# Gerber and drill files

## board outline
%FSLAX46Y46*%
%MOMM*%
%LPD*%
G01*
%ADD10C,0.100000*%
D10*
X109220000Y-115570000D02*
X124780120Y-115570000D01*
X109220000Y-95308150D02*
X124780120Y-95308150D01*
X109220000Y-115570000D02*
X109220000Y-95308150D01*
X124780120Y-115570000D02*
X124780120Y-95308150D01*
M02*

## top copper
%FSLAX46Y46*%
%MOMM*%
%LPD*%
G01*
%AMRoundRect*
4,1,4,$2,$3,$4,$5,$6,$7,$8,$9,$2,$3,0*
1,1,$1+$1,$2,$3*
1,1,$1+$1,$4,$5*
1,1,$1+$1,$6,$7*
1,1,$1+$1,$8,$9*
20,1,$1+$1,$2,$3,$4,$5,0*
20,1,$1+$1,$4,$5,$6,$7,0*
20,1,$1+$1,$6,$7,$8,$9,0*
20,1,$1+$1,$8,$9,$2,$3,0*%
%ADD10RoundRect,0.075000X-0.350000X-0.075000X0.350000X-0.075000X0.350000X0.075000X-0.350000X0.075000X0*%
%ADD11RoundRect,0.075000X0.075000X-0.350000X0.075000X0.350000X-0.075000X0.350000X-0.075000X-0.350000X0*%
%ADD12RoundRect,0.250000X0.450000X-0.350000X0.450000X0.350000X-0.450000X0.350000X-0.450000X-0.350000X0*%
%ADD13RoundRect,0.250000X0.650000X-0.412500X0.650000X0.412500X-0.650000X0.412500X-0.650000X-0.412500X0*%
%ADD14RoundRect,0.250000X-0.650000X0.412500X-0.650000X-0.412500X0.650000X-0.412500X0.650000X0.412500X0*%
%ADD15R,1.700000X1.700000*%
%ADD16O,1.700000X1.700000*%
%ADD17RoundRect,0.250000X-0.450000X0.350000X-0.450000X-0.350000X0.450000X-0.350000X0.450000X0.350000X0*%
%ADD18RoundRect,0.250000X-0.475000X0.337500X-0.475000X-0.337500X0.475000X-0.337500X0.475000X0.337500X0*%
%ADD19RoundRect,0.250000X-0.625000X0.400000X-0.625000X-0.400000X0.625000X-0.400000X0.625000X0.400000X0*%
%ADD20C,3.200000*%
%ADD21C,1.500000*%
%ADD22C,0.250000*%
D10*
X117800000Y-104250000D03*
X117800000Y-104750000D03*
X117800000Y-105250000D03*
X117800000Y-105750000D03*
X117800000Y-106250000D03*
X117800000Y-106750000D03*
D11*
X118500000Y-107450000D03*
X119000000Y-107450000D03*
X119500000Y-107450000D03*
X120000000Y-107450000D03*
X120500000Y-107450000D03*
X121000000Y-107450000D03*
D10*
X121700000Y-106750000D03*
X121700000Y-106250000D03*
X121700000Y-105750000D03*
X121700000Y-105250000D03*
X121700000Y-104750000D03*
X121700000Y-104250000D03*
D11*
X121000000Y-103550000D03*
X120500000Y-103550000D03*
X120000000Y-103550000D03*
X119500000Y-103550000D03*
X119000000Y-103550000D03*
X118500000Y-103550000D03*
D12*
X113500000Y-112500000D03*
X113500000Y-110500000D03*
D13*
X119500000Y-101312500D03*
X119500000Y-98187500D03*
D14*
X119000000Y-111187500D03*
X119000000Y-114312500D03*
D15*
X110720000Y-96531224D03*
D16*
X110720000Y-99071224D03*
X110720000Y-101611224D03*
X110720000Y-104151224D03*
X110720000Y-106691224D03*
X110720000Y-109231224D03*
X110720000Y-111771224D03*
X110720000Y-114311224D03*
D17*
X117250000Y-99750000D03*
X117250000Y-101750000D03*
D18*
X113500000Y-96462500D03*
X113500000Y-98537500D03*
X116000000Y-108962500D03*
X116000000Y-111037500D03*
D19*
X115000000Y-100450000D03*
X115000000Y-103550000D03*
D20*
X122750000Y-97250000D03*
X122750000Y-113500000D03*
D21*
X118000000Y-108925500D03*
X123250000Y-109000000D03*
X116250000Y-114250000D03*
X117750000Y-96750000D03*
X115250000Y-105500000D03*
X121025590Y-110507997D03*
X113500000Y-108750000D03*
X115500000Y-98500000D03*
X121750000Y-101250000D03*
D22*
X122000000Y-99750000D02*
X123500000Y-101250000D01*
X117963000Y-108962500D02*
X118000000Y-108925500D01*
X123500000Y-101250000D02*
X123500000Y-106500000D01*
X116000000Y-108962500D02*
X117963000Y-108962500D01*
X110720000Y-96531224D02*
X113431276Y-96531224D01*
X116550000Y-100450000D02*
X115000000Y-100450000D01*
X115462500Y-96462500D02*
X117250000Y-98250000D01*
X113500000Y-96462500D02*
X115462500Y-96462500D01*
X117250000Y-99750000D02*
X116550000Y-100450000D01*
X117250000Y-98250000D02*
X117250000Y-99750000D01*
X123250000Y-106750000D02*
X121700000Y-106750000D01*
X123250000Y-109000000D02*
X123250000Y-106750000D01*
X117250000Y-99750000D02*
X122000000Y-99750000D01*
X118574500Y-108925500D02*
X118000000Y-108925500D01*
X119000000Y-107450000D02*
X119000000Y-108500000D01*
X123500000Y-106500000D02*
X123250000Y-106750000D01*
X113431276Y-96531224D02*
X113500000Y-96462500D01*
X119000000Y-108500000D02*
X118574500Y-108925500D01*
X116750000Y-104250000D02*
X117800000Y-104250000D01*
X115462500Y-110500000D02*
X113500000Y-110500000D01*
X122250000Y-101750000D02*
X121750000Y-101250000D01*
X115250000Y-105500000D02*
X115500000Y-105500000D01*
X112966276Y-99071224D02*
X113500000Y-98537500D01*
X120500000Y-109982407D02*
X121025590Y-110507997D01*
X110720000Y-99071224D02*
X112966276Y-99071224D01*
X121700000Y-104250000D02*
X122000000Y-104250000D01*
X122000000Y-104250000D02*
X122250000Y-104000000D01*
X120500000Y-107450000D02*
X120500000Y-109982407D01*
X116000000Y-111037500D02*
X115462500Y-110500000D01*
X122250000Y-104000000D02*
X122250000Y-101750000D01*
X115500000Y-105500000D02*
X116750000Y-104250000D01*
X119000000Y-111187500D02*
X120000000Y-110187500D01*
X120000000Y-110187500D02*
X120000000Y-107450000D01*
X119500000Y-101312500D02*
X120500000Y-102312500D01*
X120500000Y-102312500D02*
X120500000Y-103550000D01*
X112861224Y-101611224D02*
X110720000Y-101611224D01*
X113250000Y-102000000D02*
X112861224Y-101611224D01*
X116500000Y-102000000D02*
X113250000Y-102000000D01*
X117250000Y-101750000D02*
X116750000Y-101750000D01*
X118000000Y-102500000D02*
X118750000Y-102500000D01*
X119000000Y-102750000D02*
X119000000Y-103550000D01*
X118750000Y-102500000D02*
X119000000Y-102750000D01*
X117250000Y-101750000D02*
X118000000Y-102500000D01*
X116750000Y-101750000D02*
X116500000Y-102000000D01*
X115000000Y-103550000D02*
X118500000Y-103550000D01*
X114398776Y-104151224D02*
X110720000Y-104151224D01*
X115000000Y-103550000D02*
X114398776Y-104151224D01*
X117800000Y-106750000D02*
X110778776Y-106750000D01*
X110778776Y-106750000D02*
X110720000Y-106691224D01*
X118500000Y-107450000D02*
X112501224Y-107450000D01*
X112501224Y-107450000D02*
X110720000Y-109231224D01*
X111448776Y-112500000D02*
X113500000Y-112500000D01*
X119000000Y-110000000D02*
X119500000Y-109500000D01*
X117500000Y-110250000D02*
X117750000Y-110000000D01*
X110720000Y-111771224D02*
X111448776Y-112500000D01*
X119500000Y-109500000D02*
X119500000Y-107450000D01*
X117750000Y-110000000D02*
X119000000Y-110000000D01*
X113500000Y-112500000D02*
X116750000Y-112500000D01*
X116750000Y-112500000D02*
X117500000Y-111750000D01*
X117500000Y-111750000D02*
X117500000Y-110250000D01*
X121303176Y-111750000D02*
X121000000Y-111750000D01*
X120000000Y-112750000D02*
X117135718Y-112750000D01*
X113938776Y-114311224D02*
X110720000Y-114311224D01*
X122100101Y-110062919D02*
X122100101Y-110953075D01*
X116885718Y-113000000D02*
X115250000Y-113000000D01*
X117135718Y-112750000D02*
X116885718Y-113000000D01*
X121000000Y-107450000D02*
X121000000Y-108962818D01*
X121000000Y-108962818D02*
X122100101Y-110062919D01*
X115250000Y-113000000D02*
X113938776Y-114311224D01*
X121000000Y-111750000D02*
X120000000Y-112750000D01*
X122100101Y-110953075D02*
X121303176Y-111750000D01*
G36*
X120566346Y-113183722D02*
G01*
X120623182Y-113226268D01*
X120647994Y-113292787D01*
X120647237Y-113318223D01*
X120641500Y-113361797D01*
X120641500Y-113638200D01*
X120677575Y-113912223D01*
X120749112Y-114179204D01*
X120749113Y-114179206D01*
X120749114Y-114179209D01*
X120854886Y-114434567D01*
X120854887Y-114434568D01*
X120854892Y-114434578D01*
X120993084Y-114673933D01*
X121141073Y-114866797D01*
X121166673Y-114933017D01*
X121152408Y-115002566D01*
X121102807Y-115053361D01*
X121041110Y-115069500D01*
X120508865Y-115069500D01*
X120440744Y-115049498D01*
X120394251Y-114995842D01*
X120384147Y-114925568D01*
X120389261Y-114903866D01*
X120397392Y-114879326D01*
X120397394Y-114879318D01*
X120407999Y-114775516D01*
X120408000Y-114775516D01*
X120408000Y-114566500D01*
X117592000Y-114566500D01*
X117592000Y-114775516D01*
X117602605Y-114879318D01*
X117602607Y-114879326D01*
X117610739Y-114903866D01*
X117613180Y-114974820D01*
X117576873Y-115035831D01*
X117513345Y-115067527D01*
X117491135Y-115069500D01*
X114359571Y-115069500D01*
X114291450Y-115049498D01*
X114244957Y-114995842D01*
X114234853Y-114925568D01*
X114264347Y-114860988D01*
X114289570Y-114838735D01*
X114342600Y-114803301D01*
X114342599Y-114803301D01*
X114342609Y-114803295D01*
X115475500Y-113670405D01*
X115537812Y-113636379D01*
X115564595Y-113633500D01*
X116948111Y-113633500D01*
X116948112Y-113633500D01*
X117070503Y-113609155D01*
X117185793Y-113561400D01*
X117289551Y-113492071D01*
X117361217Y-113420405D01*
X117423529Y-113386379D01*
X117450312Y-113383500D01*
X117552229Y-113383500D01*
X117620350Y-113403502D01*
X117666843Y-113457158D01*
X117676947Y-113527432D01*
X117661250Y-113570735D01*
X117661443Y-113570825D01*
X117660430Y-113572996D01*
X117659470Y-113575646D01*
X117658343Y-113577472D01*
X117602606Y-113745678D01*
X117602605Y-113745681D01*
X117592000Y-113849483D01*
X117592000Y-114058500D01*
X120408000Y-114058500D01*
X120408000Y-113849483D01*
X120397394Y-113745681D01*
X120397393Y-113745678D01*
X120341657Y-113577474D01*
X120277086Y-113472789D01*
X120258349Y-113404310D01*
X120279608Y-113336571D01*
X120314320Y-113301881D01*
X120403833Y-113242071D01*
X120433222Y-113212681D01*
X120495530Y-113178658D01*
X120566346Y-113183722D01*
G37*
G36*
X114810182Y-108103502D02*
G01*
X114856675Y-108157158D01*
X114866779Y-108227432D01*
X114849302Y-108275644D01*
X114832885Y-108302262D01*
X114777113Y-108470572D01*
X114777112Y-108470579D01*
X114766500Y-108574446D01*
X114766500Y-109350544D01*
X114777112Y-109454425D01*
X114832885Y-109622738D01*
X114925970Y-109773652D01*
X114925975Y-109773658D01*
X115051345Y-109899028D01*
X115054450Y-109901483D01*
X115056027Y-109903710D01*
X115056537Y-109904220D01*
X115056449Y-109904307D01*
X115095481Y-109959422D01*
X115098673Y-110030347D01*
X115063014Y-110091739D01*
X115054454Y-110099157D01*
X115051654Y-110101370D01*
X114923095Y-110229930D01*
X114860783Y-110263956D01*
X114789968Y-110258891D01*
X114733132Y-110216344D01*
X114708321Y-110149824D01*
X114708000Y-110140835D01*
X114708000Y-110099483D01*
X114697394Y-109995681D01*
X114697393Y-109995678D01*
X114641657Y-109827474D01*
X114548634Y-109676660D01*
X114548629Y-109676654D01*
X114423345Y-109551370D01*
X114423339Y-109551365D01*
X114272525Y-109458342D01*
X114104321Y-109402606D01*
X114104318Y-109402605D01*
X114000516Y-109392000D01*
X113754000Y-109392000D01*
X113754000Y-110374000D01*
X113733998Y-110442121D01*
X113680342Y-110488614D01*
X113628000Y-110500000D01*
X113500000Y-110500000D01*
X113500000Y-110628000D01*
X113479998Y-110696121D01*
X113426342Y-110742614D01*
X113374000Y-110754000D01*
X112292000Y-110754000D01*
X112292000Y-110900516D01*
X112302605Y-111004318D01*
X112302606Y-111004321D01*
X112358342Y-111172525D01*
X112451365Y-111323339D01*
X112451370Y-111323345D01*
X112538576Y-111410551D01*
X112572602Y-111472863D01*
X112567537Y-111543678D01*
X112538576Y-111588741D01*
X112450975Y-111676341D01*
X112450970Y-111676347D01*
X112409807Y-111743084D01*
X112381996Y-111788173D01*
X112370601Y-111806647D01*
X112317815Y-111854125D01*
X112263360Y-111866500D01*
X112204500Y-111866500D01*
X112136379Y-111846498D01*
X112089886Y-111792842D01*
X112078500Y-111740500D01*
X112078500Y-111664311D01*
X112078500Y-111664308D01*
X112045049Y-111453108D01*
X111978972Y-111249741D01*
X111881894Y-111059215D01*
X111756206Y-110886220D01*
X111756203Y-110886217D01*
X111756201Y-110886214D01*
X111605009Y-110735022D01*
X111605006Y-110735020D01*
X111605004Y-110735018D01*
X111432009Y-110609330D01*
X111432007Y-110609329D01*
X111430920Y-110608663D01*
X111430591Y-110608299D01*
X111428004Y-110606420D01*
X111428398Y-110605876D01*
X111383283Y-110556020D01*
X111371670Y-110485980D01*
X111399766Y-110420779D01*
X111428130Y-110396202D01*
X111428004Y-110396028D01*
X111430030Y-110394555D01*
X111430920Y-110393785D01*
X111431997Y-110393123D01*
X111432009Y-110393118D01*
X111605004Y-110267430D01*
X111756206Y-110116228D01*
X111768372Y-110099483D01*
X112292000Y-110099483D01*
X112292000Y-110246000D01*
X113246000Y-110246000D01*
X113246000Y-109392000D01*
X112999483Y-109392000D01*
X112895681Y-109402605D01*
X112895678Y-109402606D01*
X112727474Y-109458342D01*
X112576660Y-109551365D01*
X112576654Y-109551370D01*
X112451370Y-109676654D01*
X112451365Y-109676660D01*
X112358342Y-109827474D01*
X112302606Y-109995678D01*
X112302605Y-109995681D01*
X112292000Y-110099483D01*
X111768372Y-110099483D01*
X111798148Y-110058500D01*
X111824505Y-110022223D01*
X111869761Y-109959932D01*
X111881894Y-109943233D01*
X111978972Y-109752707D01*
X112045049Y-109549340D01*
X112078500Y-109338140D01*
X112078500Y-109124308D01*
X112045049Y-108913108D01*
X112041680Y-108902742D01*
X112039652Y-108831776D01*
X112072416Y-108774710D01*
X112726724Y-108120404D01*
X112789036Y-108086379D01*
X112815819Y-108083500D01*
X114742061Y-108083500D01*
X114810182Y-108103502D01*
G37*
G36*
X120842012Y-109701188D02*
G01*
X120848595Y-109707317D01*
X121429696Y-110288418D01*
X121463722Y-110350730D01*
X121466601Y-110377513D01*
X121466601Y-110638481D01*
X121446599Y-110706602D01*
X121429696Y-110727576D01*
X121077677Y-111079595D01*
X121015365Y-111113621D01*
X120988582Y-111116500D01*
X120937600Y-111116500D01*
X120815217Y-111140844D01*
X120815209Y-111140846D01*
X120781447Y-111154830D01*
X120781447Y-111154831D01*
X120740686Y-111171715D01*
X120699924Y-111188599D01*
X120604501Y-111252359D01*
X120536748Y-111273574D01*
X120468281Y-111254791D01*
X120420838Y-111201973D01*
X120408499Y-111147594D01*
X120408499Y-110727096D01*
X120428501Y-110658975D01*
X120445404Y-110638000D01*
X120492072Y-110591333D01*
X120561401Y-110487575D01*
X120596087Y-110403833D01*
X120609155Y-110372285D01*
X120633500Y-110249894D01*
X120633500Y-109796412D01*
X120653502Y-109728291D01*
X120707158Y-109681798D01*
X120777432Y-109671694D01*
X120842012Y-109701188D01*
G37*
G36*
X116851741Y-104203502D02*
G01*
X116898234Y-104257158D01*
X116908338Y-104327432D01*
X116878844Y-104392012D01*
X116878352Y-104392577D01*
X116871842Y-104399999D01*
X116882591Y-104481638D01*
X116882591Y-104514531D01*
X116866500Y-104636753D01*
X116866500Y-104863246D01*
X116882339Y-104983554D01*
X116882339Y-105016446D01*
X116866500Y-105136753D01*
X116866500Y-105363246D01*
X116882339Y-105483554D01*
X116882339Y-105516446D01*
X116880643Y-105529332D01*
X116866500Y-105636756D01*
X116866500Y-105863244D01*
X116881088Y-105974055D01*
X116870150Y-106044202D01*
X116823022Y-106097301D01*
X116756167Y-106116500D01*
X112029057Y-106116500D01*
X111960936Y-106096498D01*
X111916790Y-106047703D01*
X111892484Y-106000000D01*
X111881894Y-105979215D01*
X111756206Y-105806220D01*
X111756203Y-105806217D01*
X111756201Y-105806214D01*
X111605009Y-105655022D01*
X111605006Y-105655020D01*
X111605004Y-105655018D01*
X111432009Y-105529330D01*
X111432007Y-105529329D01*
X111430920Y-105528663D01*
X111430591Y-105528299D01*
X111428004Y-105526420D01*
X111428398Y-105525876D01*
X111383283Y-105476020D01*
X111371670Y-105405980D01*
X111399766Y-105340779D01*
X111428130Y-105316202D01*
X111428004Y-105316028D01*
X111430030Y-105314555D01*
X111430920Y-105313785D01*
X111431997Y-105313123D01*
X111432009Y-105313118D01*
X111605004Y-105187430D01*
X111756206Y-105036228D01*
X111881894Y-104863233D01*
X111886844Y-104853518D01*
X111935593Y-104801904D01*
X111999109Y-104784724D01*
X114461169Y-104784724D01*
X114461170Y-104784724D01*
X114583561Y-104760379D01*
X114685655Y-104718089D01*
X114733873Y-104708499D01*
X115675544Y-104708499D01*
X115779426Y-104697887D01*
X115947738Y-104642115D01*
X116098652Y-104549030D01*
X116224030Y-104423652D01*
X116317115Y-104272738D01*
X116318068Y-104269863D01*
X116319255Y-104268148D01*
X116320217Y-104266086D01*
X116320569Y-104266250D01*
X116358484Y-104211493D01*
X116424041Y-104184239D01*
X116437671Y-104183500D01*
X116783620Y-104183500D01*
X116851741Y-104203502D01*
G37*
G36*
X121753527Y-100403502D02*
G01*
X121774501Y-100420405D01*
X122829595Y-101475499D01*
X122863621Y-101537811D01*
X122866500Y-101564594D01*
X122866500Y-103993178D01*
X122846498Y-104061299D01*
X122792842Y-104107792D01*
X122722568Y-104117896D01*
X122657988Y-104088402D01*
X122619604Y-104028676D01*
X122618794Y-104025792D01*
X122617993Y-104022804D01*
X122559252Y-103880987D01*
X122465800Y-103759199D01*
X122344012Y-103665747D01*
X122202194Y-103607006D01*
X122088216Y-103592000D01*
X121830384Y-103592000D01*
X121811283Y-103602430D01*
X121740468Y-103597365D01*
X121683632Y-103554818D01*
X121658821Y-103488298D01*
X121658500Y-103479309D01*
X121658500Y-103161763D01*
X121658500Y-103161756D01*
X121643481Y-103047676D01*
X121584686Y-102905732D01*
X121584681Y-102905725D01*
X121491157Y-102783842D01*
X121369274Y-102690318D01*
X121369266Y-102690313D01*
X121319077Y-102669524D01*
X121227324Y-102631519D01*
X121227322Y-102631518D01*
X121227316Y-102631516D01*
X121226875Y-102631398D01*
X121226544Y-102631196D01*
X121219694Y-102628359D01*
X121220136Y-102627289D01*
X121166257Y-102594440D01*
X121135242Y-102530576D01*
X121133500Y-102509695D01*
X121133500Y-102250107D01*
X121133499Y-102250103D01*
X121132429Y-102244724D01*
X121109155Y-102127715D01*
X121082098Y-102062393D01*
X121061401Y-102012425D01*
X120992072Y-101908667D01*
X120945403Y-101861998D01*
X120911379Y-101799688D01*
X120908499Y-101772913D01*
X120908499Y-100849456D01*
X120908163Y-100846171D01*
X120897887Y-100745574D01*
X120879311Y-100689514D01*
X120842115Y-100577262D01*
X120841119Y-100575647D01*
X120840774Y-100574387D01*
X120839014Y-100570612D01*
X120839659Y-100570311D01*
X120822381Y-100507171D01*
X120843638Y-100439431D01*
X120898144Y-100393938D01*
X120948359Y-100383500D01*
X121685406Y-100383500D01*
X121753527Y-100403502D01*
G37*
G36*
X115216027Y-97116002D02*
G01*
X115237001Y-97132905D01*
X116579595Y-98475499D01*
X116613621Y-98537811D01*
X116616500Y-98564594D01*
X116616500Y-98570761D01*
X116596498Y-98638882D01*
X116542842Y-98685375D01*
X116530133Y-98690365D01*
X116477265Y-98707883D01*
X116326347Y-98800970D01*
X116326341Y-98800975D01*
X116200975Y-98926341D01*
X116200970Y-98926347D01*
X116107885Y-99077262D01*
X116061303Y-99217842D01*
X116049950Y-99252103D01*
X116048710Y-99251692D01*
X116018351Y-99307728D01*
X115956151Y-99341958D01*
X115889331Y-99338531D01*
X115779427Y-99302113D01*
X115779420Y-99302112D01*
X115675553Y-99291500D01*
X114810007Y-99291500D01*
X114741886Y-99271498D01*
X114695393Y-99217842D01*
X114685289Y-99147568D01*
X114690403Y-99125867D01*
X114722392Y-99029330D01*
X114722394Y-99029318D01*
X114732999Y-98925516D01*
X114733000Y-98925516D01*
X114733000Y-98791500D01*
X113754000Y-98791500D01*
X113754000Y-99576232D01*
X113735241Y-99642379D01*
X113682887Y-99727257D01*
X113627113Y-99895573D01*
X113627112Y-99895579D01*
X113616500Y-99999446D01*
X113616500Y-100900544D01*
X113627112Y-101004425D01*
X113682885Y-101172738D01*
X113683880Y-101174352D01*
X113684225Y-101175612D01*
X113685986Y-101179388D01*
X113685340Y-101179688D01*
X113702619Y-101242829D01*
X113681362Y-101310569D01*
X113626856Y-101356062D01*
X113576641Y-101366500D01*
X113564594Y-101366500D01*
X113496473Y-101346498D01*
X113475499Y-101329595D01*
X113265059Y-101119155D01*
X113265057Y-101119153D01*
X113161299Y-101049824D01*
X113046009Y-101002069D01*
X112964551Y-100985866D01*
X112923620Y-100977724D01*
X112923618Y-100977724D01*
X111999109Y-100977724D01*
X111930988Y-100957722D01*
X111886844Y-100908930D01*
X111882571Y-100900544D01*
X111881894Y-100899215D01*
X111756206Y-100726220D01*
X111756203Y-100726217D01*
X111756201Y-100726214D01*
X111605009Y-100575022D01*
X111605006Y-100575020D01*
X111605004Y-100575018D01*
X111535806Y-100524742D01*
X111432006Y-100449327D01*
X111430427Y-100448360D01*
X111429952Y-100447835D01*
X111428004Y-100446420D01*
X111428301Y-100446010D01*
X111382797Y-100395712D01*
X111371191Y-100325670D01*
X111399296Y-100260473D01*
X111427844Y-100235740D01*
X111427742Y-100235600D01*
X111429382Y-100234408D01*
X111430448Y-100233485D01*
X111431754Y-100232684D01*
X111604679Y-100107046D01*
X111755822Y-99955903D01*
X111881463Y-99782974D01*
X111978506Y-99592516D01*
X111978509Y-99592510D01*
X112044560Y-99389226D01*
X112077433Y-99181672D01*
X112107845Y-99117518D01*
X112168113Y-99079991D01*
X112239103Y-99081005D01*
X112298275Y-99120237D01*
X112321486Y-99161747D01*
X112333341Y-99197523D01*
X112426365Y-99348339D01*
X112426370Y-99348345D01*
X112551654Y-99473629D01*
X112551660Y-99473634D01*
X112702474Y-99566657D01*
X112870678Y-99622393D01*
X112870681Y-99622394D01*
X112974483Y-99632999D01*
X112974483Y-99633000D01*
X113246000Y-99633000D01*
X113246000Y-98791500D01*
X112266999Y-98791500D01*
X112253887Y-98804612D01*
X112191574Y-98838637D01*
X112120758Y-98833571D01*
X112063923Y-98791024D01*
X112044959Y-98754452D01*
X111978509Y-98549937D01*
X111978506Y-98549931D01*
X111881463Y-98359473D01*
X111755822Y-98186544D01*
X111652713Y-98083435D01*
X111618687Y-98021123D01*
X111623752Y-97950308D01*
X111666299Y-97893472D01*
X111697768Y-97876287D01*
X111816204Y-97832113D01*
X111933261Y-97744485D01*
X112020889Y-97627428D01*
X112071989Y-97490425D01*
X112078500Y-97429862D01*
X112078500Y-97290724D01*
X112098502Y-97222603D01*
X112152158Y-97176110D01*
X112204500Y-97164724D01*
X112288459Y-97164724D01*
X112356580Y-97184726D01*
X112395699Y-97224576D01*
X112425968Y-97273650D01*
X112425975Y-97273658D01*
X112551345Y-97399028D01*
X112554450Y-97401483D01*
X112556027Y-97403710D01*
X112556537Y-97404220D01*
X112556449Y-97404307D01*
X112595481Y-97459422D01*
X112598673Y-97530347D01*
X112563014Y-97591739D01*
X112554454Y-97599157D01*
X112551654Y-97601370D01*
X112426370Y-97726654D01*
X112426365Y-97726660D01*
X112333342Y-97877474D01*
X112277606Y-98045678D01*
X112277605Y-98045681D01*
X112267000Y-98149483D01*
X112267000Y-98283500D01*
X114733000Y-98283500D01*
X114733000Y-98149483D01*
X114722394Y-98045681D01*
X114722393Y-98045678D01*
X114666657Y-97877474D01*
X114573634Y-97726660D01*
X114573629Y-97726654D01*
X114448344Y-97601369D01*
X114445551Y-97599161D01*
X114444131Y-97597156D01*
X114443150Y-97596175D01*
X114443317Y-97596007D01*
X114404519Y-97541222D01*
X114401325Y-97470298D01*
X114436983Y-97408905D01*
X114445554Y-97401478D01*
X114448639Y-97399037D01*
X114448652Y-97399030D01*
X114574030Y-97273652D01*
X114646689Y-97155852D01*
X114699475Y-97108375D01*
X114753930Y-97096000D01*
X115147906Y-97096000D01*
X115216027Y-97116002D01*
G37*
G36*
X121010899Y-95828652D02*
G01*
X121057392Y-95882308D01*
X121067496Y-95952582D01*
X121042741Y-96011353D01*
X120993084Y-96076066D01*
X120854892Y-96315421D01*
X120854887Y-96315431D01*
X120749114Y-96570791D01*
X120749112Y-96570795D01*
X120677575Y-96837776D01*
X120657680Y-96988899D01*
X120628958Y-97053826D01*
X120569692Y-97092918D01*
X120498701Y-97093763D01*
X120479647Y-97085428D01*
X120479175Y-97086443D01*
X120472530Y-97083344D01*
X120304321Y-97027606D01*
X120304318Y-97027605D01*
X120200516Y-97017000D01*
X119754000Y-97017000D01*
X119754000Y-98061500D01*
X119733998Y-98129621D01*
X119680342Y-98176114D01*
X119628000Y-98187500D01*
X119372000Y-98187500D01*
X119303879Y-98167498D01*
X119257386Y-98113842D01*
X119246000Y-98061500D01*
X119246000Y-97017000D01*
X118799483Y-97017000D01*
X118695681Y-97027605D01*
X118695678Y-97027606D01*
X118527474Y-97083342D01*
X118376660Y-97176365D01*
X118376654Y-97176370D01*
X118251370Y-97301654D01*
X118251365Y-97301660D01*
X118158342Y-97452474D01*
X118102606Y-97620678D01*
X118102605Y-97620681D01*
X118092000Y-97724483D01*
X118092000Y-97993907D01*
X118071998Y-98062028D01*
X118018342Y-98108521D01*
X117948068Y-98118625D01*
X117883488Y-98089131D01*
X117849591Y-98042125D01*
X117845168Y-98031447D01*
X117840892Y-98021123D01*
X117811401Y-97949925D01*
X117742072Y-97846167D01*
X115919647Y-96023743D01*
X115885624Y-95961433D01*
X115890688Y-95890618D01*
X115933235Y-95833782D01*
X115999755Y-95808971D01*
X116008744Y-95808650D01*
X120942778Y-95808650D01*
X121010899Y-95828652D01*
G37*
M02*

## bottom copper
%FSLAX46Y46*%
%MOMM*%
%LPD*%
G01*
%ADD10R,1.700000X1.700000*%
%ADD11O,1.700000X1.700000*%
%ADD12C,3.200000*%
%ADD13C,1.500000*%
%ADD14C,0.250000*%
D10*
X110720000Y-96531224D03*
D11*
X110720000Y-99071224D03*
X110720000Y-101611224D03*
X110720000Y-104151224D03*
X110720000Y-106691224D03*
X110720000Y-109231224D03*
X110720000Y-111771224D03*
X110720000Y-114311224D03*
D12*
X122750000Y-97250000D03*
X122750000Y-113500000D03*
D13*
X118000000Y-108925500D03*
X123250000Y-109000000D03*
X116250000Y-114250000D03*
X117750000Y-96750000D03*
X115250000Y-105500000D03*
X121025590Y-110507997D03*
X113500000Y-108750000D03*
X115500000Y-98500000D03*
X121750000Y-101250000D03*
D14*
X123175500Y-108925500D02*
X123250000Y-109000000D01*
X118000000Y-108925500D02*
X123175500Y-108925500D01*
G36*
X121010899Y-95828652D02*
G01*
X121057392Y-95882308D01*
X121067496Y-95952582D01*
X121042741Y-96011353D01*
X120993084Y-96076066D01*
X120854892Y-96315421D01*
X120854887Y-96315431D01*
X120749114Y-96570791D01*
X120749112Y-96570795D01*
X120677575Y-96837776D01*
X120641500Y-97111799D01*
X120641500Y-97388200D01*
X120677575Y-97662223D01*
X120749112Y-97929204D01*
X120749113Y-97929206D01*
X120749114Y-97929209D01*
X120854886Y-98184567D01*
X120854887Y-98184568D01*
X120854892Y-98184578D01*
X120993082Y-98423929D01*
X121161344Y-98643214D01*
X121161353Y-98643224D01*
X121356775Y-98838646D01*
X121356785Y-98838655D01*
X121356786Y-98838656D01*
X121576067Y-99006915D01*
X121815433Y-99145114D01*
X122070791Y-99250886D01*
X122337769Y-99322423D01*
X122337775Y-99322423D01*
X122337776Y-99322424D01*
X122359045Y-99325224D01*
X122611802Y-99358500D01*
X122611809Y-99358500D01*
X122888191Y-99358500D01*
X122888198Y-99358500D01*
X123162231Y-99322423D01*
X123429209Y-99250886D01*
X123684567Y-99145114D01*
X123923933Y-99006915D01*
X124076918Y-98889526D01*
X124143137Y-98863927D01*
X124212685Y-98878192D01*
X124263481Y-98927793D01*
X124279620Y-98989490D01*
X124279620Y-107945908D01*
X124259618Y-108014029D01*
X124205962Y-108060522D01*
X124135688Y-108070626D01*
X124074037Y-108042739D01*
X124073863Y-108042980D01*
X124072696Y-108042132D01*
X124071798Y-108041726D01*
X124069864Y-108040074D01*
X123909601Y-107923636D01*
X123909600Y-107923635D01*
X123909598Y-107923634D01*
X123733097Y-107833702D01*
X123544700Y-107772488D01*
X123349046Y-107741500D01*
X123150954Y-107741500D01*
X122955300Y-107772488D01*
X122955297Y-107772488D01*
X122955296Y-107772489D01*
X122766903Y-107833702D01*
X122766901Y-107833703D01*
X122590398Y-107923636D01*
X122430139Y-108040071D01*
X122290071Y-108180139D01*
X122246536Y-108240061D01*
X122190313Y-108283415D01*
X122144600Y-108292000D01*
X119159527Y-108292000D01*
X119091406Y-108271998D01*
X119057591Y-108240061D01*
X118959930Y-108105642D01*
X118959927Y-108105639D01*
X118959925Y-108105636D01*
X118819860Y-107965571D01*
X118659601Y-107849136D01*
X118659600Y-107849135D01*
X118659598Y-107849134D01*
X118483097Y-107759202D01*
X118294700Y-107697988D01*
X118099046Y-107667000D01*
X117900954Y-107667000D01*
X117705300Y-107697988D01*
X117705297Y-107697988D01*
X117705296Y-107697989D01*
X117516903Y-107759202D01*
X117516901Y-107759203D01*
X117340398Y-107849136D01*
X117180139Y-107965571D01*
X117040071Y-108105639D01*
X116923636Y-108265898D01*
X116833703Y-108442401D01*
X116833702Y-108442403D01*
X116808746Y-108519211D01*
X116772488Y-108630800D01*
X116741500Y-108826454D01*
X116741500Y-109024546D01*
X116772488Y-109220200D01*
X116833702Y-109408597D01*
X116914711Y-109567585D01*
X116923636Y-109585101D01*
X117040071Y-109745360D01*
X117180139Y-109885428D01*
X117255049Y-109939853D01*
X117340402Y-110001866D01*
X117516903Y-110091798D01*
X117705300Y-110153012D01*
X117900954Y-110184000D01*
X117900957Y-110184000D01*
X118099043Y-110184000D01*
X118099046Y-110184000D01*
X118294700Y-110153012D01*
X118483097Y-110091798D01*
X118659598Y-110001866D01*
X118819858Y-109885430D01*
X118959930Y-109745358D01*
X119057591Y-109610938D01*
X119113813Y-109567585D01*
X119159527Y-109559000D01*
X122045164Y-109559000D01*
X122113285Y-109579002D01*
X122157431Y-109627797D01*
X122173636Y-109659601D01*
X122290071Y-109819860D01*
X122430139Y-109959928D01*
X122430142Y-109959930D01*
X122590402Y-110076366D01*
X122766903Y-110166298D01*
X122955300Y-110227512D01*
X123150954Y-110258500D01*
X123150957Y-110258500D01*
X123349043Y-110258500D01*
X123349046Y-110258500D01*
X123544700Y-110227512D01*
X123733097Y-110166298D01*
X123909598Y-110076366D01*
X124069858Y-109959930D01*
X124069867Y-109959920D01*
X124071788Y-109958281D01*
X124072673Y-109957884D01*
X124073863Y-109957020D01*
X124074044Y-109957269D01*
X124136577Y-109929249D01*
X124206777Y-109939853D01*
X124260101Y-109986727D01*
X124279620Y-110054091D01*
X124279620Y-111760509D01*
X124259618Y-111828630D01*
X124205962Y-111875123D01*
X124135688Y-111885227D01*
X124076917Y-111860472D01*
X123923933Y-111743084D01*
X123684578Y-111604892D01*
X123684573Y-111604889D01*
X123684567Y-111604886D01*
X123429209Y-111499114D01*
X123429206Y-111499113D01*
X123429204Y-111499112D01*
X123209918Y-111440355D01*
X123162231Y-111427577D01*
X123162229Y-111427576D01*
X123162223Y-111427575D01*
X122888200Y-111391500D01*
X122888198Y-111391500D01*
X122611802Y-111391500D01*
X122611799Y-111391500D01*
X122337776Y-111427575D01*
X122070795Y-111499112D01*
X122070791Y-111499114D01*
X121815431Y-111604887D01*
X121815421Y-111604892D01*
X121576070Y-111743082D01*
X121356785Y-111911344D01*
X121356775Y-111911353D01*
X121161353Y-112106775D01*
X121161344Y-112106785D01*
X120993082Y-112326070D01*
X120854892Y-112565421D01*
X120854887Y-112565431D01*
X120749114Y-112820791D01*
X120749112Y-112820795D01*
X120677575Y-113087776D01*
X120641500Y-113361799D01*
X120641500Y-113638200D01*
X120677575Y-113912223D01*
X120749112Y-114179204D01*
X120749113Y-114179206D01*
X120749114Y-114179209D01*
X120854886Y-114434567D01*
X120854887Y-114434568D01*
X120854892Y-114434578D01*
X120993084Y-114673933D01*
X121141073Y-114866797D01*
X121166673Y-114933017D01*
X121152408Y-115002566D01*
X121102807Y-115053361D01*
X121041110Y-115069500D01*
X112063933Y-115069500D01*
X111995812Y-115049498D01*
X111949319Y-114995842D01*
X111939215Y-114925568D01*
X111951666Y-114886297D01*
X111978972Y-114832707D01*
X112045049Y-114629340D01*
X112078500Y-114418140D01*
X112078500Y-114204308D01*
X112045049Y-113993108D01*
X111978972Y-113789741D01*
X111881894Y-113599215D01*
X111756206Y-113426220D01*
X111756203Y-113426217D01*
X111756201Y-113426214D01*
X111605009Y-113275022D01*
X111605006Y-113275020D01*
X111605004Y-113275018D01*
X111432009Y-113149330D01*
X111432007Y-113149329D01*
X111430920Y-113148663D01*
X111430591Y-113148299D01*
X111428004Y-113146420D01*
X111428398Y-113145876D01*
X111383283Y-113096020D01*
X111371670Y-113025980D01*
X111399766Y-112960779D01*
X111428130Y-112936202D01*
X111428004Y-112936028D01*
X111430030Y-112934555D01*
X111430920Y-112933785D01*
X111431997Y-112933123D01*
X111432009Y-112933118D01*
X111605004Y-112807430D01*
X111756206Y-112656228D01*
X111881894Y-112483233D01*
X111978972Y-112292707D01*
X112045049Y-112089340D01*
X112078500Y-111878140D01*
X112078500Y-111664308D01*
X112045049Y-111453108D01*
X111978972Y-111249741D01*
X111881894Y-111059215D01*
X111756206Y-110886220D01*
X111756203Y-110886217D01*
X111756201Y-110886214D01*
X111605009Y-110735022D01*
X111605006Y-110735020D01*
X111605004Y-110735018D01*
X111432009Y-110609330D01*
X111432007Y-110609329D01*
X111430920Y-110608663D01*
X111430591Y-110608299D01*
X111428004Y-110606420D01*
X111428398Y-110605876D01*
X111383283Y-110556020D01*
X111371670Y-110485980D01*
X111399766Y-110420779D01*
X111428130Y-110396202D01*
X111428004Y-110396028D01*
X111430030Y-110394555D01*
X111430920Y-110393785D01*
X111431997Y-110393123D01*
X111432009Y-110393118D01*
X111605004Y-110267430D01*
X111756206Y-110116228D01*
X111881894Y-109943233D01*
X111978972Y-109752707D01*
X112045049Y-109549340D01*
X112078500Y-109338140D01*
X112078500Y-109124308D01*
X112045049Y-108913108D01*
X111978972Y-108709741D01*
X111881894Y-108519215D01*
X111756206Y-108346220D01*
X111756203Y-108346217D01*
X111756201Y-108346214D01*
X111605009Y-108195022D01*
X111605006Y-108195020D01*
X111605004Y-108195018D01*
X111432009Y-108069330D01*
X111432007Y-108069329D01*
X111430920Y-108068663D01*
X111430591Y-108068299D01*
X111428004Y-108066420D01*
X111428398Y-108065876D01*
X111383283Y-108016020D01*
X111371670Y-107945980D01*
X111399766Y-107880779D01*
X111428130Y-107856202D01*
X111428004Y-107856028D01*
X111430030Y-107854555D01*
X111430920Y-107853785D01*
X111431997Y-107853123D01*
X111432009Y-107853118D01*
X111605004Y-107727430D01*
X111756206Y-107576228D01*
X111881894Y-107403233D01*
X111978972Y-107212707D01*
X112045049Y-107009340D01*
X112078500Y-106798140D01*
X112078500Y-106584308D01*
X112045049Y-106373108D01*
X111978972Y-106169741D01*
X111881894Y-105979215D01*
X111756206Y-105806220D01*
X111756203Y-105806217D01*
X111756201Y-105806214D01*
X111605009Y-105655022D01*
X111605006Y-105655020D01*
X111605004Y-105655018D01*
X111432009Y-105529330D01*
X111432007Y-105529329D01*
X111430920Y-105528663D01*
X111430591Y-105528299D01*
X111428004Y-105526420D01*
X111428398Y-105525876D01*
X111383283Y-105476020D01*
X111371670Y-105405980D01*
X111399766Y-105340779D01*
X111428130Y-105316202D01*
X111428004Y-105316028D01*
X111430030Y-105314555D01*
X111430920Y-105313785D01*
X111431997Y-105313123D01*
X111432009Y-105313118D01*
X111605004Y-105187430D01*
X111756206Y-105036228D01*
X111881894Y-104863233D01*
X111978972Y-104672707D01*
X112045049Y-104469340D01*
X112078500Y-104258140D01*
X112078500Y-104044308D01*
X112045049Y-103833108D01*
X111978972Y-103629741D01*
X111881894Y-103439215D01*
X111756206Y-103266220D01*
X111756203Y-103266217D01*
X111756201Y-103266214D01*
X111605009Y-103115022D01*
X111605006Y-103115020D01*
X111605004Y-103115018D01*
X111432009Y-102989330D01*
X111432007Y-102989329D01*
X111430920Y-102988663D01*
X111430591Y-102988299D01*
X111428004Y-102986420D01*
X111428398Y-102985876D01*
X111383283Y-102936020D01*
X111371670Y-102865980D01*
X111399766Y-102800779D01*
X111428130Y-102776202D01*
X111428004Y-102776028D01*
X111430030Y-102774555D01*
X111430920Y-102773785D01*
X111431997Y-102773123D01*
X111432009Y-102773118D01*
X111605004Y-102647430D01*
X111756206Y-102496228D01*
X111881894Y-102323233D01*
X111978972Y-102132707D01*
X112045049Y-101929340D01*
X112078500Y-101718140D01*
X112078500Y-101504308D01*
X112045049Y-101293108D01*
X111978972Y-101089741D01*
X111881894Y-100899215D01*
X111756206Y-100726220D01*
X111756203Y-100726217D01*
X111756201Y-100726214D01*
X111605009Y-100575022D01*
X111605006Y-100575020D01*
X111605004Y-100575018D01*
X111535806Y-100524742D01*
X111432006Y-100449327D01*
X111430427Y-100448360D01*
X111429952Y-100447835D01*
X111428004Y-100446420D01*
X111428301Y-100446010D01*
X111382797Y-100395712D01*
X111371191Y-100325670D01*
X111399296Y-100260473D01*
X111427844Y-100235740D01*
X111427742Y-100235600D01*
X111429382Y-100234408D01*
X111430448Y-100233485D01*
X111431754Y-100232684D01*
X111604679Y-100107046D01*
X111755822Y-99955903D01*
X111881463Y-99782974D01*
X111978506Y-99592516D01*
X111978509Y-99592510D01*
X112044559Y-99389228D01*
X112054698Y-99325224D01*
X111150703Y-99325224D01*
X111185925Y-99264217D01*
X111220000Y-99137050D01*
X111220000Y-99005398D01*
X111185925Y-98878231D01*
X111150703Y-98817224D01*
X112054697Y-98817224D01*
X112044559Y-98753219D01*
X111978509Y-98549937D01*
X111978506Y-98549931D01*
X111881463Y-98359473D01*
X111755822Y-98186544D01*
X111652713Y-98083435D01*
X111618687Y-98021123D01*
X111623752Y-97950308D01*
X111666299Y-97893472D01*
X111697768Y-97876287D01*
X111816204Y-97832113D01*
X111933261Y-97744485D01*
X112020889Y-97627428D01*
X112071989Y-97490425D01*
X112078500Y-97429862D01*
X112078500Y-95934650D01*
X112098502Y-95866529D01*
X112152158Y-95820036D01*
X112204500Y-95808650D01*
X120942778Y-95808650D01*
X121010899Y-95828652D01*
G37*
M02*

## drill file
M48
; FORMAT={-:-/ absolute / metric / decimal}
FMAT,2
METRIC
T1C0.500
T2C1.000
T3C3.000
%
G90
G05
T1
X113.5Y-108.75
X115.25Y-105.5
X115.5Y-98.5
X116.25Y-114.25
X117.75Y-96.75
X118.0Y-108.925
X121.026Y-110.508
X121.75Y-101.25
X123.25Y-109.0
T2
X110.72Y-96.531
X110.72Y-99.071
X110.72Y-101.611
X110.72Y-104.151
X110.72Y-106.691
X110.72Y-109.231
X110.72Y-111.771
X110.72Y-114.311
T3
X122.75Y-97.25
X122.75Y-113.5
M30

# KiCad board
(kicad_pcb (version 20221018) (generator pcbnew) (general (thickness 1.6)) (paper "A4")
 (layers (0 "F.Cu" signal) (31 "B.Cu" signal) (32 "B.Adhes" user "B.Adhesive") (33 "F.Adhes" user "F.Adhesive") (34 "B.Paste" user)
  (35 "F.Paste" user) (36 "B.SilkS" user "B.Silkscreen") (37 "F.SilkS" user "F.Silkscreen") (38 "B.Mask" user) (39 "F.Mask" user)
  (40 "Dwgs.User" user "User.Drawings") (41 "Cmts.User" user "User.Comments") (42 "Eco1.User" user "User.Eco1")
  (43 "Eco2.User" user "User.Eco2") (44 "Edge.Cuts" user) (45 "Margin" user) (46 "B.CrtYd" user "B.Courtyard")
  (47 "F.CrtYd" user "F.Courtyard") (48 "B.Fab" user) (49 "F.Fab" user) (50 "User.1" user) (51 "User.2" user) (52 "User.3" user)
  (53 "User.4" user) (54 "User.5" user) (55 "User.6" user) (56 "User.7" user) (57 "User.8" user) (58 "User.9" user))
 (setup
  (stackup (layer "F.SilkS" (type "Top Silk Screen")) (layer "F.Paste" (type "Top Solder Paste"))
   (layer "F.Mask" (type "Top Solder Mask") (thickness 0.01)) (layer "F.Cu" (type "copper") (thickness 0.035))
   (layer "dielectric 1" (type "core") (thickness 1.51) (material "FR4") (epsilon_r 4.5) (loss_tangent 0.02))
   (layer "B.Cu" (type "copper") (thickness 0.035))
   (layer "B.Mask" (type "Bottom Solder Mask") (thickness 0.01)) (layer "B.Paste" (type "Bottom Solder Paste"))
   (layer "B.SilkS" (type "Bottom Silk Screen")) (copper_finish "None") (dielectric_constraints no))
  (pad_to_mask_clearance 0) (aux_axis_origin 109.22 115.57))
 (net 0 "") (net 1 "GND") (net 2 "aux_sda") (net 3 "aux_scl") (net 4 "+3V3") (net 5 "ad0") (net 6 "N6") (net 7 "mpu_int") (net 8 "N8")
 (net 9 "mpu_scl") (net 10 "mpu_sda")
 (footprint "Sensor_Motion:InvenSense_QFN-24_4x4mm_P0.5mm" (layer "F.Cu") (at 119.75 105.5)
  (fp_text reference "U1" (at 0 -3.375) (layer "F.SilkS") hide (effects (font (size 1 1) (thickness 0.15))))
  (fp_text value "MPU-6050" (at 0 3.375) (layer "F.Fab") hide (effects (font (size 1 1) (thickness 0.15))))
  (pad "1" smd roundrect (at -1.95 -1.25) (size 0.85 0.3) (layers "F.Cu" "F.Paste" "F.Mask") (roundrect_rratio 0.25) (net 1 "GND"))
  (pad "2" smd roundrect (at -1.95 -0.75) (size 0.85 0.3) (layers "F.Cu" "F.Paste" "F.Mask") (roundrect_rratio 0.25))
  (pad "3" smd roundrect (at -1.95 -0.25) (size 0.85 0.3) (layers "F.Cu" "F.Paste" "F.Mask") (roundrect_rratio 0.25))
  (pad "4" smd roundrect (at -1.95 0.25) (size 0.85 0.3) (layers "F.Cu" "F.Paste" "F.Mask") (roundrect_rratio 0.25))
  (pad "5" smd roundrect (at -1.95 0.75) (size 0.85 0.3) (layers "F.Cu" "F.Paste" "F.Mask") (roundrect_rratio 0.25))
  (pad "6" smd roundrect (at -1.95 1.25) (size 0.85 0.3) (layers "F.Cu" "F.Paste" "F.Mask") (roundrect_rratio 0.25) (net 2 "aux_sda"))
  (pad "7" smd roundrect (at -1.25 1.95 90) (size 0.85 0.3) (layers "F.Cu" "F.Paste" "F.Mask") (roundrect_rratio 0.25) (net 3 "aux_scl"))
  (pad "8" smd roundrect (at -0.75 1.95 90) (size 0.85 0.3) (layers "F.Cu" "F.Paste" "F.Mask") (roundrect_rratio 0.25) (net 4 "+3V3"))
  (pad "9" smd roundrect (at -0.25 1.95 90) (size 0.85 0.3) (layers "F.Cu" "F.Paste" "F.Mask") (roundrect_rratio 0.25) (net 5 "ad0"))
  (pad "10" smd roundrect (at 0.25 1.95 90) (size 0.85 0.3) (layers "F.Cu" "F.Paste" "F.Mask") (roundrect_rratio 0.25) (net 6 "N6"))
  (pad "11" smd roundrect (at 0.75 1.95 90) (size 0.85 0.3) (layers "F.Cu" "F.Paste" "F.Mask") (roundrect_rratio 0.25) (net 1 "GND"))
  (pad "12" smd roundrect (at 1.25 1.95 90) (size 0.85 0.3) (layers "F.Cu" "F.Paste" "F.Mask") (roundrect_rratio 0.25) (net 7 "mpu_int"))
  (pad "13" smd roundrect (at 1.95 1.25) (size 0.85 0.3) (layers "F.Cu" "F.Paste" "F.Mask") (roundrect_rratio 0.25) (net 4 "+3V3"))
  (pad "14" smd roundrect (at 1.95 0.75) (size 0.85 0.3) (layers "F.Cu" "F.Paste" "F.Mask") (roundrect_rratio 0.25))
  (pad "15" smd roundrect (at 1.95 0.25) (size 0.85 0.3) (layers "F.Cu" "F.Paste" "F.Mask") (roundrect_rratio 0.25))
  (pad "16" smd roundrect (at 1.95 -0.25) (size 0.85 0.3) (layers "F.Cu" "F.Paste" "F.Mask") (roundrect_rratio 0.25))
  (pad "17" smd roundrect (at 1.95 -0.75) (size 0.85 0.3) (layers "F.Cu" "F.Paste" "F.Mask") (roundrect_rratio 0.25))
  (pad "18" smd roundrect (at 1.95 -1.25) (size 0.85 0.3) (layers "F.Cu" "F.Paste" "F.Mask") (roundrect_rratio 0.25) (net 1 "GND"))
  (pad "19" smd roundrect (at 1.25 -1.95 90) (size 0.85 0.3) (layers "F.Cu" "F.Paste" "F.Mask") (roundrect_rratio 0.25))
  (pad "20" smd roundrect (at 0.75 -1.95 90) (size 0.85 0.3) (layers "F.Cu" "F.Paste" "F.Mask") (roundrect_rratio 0.25) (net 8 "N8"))
  (pad "21" smd roundrect (at 0.25 -1.95 90) (size 0.85 0.3) (layers "F.Cu" "F.Paste" "F.Mask") (roundrect_rratio 0.25))
  (pad "22" smd roundrect (at -0.25 -1.95 90) (size 0.85 0.3) (layers "F.Cu" "F.Paste" "F.Mask") (roundrect_rratio 0.25))
  (pad "23" smd roundrect (at -0.75 -1.95 90) (size 0.85 0.3) (layers "F.Cu" "F.Paste" "F.Mask") (roundrect_rratio 0.25) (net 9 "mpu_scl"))
  (pad "24" smd roundrect (at -1.25 -1.95 90) (size 0.85 0.3) (layers "F.Cu" "F.Paste" "F.Mask") (roundrect_rratio 0.25) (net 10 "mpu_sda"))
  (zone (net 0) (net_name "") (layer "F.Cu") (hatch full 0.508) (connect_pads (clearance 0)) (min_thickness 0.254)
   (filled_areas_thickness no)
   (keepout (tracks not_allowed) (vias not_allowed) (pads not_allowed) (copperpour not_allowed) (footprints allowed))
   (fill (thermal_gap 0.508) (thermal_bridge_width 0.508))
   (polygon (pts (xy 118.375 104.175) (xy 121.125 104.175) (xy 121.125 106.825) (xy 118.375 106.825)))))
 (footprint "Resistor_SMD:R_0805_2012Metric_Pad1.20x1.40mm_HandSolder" (layer "F.Cu") (at 113.5 111.5 90)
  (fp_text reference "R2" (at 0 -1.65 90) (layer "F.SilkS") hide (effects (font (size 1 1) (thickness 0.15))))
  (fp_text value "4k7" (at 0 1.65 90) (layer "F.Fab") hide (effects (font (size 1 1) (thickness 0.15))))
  (pad "1" smd roundrect (at -1 0 90) (size 1.2 1.4) (layers "F.Cu" "F.Paste" "F.Mask") (roundrect_rratio 0.208333) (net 5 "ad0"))
  (pad "2" smd roundrect (at 1 0 90) (size 1.2 1.4) (layers "F.Cu" "F.Paste" "F.Mask") (roundrect_rratio 0.208333) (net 1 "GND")))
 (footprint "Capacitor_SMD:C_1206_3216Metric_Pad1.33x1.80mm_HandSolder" (layer "F.Cu") (at 119.5 99.75 90)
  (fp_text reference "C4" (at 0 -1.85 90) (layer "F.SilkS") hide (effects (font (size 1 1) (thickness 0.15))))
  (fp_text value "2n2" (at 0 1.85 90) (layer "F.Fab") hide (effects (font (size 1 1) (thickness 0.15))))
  (pad "1" smd roundrect (at -1.5625 0 90) (size 1.325 1.8) (layers "F.Cu" "F.Paste" "F.Mask") (roundrect_rratio 0.188679) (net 8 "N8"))
  (pad "2" smd roundrect (at 1.5625 0 90) (size 1.325 1.8) (layers "F.Cu" "F.Paste" "F.Mask") (roundrect_rratio 0.188679) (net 1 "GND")))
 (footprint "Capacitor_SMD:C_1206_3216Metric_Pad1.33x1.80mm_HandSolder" (layer "F.Cu") (at 119 112.75 -90)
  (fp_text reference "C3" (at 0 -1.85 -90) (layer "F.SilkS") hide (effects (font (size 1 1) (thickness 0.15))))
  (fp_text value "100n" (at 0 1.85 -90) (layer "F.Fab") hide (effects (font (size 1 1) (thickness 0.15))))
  (pad "1" smd roundrect (at -1.5625 0 270) (size 1.325 1.8) (layers "F.Cu" "F.Paste" "F.Mask") (roundrect_rratio 0.188679) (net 6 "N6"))
  (pad "2" smd roundrect (at 1.5625 0 270) (size 1.325 1.8) (layers "F.Cu" "F.Paste" "F.Mask") (roundrect_rratio 0.188679) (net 1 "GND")))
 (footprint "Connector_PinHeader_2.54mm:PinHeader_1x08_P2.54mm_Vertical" (layer "F.Cu") (at 110.72 96.531224)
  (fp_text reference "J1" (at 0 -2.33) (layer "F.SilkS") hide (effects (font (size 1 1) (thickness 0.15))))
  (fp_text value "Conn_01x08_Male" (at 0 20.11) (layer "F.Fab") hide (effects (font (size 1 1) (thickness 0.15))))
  (pad "1" thru_hole rect (at 0 0) (size 1.7 1.7) (drill 1) (layers "*.Cu" "*.Mask") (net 4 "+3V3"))
  (pad "2" thru_hole oval (at 0 2.54) (size 1.7 1.7) (drill 1) (layers "*.Cu" "*.Mask") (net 1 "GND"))
  (pad "3" thru_hole oval (at 0 5.08) (size 1.7 1.7) (drill 1) (layers "*.Cu" "*.Mask") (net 9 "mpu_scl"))
  (pad "4" thru_hole oval (at 0 7.62) (size 1.7 1.7) (drill 1) (layers "*.Cu" "*.Mask") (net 10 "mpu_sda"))
  (pad "5" thru_hole oval (at 0 10.16) (size 1.7 1.7) (drill 1) (layers "*.Cu" "*.Mask") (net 2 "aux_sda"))
  (pad "6" thru_hole oval (at 0 12.7) (size 1.7 1.7) (drill 1) (layers "*.Cu" "*.Mask") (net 3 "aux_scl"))
  (pad "7" thru_hole oval (at 0 15.24) (size 1.7 1.7) (drill 1) (layers "*.Cu" "*.Mask") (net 5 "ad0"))
  (pad "8" thru_hole oval (at 0 17.78) (size 1.7 1.7) (drill 1) (layers "*.Cu" "*.Mask") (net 7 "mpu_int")))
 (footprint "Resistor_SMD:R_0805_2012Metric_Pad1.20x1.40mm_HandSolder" (layer "F.Cu") (at 117.25 100.75 -90)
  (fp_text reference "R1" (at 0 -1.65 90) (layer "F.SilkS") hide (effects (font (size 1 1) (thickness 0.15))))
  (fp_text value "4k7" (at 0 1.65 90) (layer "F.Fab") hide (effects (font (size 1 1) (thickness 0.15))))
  (pad "1" smd roundrect (at -1 0 270) (size 1.2 1.4) (layers "F.Cu" "F.Paste" "F.Mask") (roundrect_rratio 0.208333) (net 4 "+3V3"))
  (pad "2" smd roundrect (at 1 0 270) (size 1.2 1.4) (layers "F.Cu" "F.Paste" "F.Mask") (roundrect_rratio 0.208333) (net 9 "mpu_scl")))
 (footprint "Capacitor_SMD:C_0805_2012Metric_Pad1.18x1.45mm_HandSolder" (layer "F.Cu") (at 113.5 97.5 -90)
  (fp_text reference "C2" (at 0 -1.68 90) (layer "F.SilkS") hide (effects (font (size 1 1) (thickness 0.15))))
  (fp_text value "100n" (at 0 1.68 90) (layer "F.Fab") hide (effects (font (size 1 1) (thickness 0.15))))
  (pad "1" smd roundrect (at -1.0375 0 270) (size 1.175 1.45) (layers "F.Cu" "F.Paste" "F.Mask") (roundrect_rratio 0.212766) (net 4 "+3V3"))
  (pad "2" smd roundrect (at 1.0375 0 270) (size 1.175 1.45) (layers "F.Cu" "F.Paste" "F.Mask") (roundrect_rratio 0.212766) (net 1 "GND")))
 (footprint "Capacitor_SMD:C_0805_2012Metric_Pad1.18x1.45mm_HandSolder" (layer "F.Cu") (at 116 110 -90)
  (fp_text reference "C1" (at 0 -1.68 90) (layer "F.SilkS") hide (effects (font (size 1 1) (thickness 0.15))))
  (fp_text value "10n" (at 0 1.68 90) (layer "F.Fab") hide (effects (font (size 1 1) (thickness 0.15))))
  (pad "1" smd roundrect (at -1.0375 0 270) (size 1.175 1.45) (layers "F.Cu" "F.Paste" "F.Mask") (roundrect_rratio 0.212766) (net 4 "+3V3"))
  (pad "2" smd roundrect (at 1.0375 0 270) (size 1.175 1.45) (layers "F.Cu" "F.Paste" "F.Mask") (roundrect_rratio 0.212766) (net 1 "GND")))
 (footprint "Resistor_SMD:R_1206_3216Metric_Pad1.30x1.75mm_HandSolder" (layer "F.Cu") (at 115 102 -90)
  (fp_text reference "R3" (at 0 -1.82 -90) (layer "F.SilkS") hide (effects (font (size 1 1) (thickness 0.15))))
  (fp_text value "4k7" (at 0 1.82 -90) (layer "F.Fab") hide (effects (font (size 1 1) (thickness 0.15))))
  (pad "1" smd roundrect (at -1.55 0 270) (size 1.3 1.75) (layers "F.Cu" "F.Paste" "F.Mask") (roundrect_rratio 0.192308) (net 4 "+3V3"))
  (pad "2" smd roundrect (at 1.55 0 270) (size 1.3 1.75) (layers "F.Cu" "F.Paste" "F.Mask") (roundrect_rratio 0.192308) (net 10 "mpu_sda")))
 (gr_line (start 109.22 115.57) (end 124.78012 115.57) (stroke (width 0.1) (type solid)) (layer "Edge.Cuts"))
 (gr_line (start 109.22 95.30815) (end 124.78012 95.30815) (stroke (width 0.1) (type solid)) (layer "Edge.Cuts"))
 (gr_line (start 109.22 115.57) (end 109.22 95.30815) (stroke (width 0.1) (type solid)) (layer "Edge.Cuts"))
 (gr_line (start 124.78012 115.57) (end 124.78012 95.30815) (stroke (width 0.1) (type solid)) (layer "Edge.Cuts"))
 (via (at 122.75 97.25) (size 3.2) (drill 3) (layers "F.Cu" "B.Cu") (free) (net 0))
 (via (at 122.75 113.5) (size 3.2) (drill 3) (layers "F.Cu" "B.Cu") (free) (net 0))
 (segment (start 122 99.75) (end 123.5 101.25) (width 0.25) (layer "F.Cu") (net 4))
 (segment (start 117.963 108.9625) (end 118 108.9255) (width 0.25) (layer "F.Cu") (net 4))
 (segment (start 123.5 101.25) (end 123.5 106.5) (width 0.25) (layer "F.Cu") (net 4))
 (segment (start 116 108.9625) (end 117.963 108.9625) (width 0.25) (layer "F.Cu") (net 4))
 (segment (start 110.72 96.531224) (end 113.431276 96.531224) (width 0.25) (layer "F.Cu") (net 4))
 (segment (start 116.55 100.45) (end 115 100.45) (width 0.25) (layer "F.Cu") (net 4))
 (segment (start 115.4625 96.4625) (end 117.25 98.25) (width 0.25) (layer "F.Cu") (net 4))
 (segment (start 113.5 96.4625) (end 115.4625 96.4625) (width 0.25) (layer "F.Cu") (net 4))
 (segment (start 117.25 99.75) (end 116.55 100.45) (width 0.25) (layer "F.Cu") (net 4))
 (segment (start 117.25 98.25) (end 117.25 99.75) (width 0.25) (layer "F.Cu") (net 4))
 (segment (start 123.25 106.75) (end 121.7 106.75) (width 0.25) (layer "F.Cu") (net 4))
 (segment (start 123.25 109) (end 123.25 106.75) (width 0.25) (layer "F.Cu") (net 4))
 (segment (start 117.25 99.75) (end 122 99.75) (width 0.25) (layer "F.Cu") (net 4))
 (segment (start 118.5745 108.9255) (end 118 108.9255) (width 0.25) (layer "F.Cu") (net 4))
 (segment (start 119 107.45) (end 119 108.5) (width 0.25) (layer "F.Cu") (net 4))
 (segment (start 123.5 106.5) (end 123.25 106.75) (width 0.25) (layer "F.Cu") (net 4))
 (segment (start 113.431276 96.531224) (end 113.5 96.4625) (width 0.25) (layer "F.Cu") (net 4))
 (segment (start 119 108.5) (end 118.5745 108.9255) (width 0.25) (layer "F.Cu") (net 4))
 (via (at 118 108.9255) (size 1.5) (drill 0.5) (layers "F.Cu" "B.Cu") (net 4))
 (via (at 123.25 109) (size 1.5) (drill 0.5) (layers "F.Cu" "B.Cu") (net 4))
 (segment (start 123.1755 108.9255) (end 123.25 109) (width 0.25) (layer "B.Cu") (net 4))
 (segment (start 118 108.9255) (end 123.1755 108.9255) (width 0.25) (layer "B.Cu") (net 4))
 (segment (start 116.75 104.25) (end 117.8 104.25) (width 0.25) (layer "F.Cu") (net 1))
 (segment (start 115.4625 110.5) (end 113.5 110.5) (width 0.25) (layer "F.Cu") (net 1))
 (segment (start 122.25 101.75) (end 121.75 101.25) (width 0.25) (layer "F.Cu") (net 1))
 (segment (start 115.25 105.5) (end 115.5 105.5) (width 0.25) (layer "F.Cu") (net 1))
 (segment (start 112.966276 99.071224) (end 113.5 98.5375) (width 0.25) (layer "F.Cu") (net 1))
 (segment (start 120.5 109.982407) (end 121.02559 110.507997) (width 0.25) (layer "F.Cu") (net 1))
 (segment (start 110.72 99.071224) (end 112.966276 99.071224) (width 0.25) (layer "F.Cu") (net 1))
 (segment (start 121.7 104.25) (end 122 104.25) (width 0.25) (layer "F.Cu") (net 1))
 (segment (start 122 104.25) (end 122.25 104) (width 0.25) (layer "F.Cu") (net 1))
 (segment (start 120.5 107.45) (end 120.5 109.982407) (width 0.25) (layer "F.Cu") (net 1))
 (segment (start 116 111.0375) (end 115.4625 110.5) (width 0.25) (layer "F.Cu") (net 1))
 (segment (start 122.25 104) (end 122.25 101.75) (width 0.25) (layer "F.Cu") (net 1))
 (segment (start 115.5 105.5) (end 116.75 104.25) (width 0.25) (layer "F.Cu") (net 1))
 (via (at 116.25 114.25) (size 1.5) (drill 0.5) (layers "F.Cu" "B.Cu") (free) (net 1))
 (via (at 117.75 96.75) (size 1.5) (drill 0.5) (layers "F.Cu" "B.Cu") (free) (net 1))
 (via (at 115.25 105.5) (size 1.5) (drill 0.5) (layers "F.Cu" "B.Cu") (free) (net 1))
 (via (at 121.02559 110.507997) (size 1.5) (drill 0.5) (layers "F.Cu" "B.Cu") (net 1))
 (via (at 113.5 108.75) (size 1.5) (drill 0.5) (layers "F.Cu" "B.Cu") (free) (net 1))
 (via (at 115.5 98.5) (size 1.5) (drill 0.5) (layers "F.Cu" "B.Cu") (free) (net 1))
 (via (at 121.75 101.25) (size 1.5) (drill 0.5) (layers "F.Cu" "B.Cu") (free) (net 1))
 (segment (start 119 111.1875) (end 120 110.1875) (width 0.25) (layer "F.Cu") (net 6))
 (segment (start 120 110.1875) (end 120 107.45) (width 0.25) (layer "F.Cu") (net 6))
 (segment (start 119.5 101.3125) (end 120.5 102.3125) (width 0.25) (layer "F.Cu") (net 8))
 (segment (start 120.5 102.3125) (end 120.5 103.55) (width 0.25) (layer "F.Cu") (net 8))
 (segment (start 112.861224 101.611224) (end 110.72 101.611224) (width 0.25) (layer "F.Cu") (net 9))
 (segment (start 113.25 102) (end 112.861224 101.611224) (width 0.25) (layer "F.Cu") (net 9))
 (segment (start 116.5 102) (end 113.25 102) (width 0.25) (layer "F.Cu") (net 9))
 (segment (start 117.25 101.75) (end 116.75 101.75) (width 0.25) (layer "F.Cu") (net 9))
 (segment (start 118 102.5) (end 118.75 102.5) (width 0.25) (layer "F.Cu") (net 9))
 (segment (start 119 102.75) (end 119 103.55) (width 0.25) (layer "F.Cu") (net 9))
 (segment (start 118.75 102.5) (end 119 102.75) (width 0.25) (layer "F.Cu") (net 9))
 (segment (start 117.25 101.75) (end 118 102.5) (width 0.25) (layer "F.Cu") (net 9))
 (segment (start 116.75 101.75) (end 116.5 102) (width 0.25) (layer "F.Cu") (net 9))
 (segment (start 115 103.55) (end 118.5 103.55) (width 0.25) (layer "F.Cu") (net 10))
 (segment (start 114.398776 104.151224) (end 110.72 104.151224) (width 0.25) (layer "F.Cu") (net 10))
 (segment (start 115 103.55) (end 114.398776 104.151224) (width 0.25) (layer "F.Cu") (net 10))
 (segment (start 117.8 106.75) (end 110.778776 106.75) (width 0.25) (layer "F.Cu") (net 2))
 (segment (start 110.778776 106.75) (end 110.72 106.691224) (width 0.25) (layer "F.Cu") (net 2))
 (segment (start 118.5 107.45) (end 112.501224 107.45) (width 0.25) (layer "F.Cu") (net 3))
 (segment (start 112.501224 107.45) (end 110.72 109.231224) (width 0.25) (layer "F.Cu") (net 3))
 (segment (start 111.448776 112.5) (end 113.5 112.5) (width 0.25) (layer "F.Cu") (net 5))
 (segment (start 119 110) (end 119.5 109.5) (width 0.25) (layer "F.Cu") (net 5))
 (segment (start 117.5 110.25) (end 117.75 110) (width 0.25) (layer "F.Cu") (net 5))
 (segment (start 110.72 111.771224) (end 111.448776 112.5) (width 0.25) (layer "F.Cu") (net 5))
 (segment (start 119.5 109.5) (end 119.5 107.45) (width 0.25) (layer "F.Cu") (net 5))
 (segment (start 117.75 110) (end 119 110) (width 0.25) (layer "F.Cu") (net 5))
 (segment (start 113.5 112.5) (end 116.75 112.5) (width 0.25) (layer "F.Cu") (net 5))
 (segment (start 116.75 112.5) (end 117.5 111.75) (width 0.25) (layer "F.Cu") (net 5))
 (segment (start 117.5 111.75) (end 117.5 110.25) (width 0.25) (layer "F.Cu") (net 5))
 (segment (start 121.303176 111.75) (end 121 111.75) (width 0.25) (layer "F.Cu") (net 7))
 (segment (start 120 112.75) (end 117.135718 112.75) (width 0.25) (layer "F.Cu") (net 7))
 (segment (start 113.938776 114.311224) (end 110.72 114.311224) (width 0.25) (layer "F.Cu") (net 7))
 (segment (start 122.100101 110.062919) (end 122.100101 110.953075) (width 0.25) (layer "F.Cu") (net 7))
 (segment (start 116.885718 113) (end 115.25 113) (width 0.25) (layer "F.Cu") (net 7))
 (segment (start 117.135718 112.75) (end 116.885718 113) (width 0.25) (layer "F.Cu") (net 7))
 (segment (start 121 107.45) (end 121 108.962818) (width 0.25) (layer "F.Cu") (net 7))
 (segment (start 121 108.962818) (end 122.100101 110.062919) (width 0.25) (layer "F.Cu") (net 7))
 (segment (start 115.25 113) (end 113.938776 114.311224) (width 0.25) (layer "F.Cu") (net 7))
 (segment (start 121 111.75) (end 120 112.75) (width 0.25) (layer "F.Cu") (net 7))
 (segment (start 122.100101 110.953075) (end 121.303176 111.75) (width 0.25) (layer "F.Cu") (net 7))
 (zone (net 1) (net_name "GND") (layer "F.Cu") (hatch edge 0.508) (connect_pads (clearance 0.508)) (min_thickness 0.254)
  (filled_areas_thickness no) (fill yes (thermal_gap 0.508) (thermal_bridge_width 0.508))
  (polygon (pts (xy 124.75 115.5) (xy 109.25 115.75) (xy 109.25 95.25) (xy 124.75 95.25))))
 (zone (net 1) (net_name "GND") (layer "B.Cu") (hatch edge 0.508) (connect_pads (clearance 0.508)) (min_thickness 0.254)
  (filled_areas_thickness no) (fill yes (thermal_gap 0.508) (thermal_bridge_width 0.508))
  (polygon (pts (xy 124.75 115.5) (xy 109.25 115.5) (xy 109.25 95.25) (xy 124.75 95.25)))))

